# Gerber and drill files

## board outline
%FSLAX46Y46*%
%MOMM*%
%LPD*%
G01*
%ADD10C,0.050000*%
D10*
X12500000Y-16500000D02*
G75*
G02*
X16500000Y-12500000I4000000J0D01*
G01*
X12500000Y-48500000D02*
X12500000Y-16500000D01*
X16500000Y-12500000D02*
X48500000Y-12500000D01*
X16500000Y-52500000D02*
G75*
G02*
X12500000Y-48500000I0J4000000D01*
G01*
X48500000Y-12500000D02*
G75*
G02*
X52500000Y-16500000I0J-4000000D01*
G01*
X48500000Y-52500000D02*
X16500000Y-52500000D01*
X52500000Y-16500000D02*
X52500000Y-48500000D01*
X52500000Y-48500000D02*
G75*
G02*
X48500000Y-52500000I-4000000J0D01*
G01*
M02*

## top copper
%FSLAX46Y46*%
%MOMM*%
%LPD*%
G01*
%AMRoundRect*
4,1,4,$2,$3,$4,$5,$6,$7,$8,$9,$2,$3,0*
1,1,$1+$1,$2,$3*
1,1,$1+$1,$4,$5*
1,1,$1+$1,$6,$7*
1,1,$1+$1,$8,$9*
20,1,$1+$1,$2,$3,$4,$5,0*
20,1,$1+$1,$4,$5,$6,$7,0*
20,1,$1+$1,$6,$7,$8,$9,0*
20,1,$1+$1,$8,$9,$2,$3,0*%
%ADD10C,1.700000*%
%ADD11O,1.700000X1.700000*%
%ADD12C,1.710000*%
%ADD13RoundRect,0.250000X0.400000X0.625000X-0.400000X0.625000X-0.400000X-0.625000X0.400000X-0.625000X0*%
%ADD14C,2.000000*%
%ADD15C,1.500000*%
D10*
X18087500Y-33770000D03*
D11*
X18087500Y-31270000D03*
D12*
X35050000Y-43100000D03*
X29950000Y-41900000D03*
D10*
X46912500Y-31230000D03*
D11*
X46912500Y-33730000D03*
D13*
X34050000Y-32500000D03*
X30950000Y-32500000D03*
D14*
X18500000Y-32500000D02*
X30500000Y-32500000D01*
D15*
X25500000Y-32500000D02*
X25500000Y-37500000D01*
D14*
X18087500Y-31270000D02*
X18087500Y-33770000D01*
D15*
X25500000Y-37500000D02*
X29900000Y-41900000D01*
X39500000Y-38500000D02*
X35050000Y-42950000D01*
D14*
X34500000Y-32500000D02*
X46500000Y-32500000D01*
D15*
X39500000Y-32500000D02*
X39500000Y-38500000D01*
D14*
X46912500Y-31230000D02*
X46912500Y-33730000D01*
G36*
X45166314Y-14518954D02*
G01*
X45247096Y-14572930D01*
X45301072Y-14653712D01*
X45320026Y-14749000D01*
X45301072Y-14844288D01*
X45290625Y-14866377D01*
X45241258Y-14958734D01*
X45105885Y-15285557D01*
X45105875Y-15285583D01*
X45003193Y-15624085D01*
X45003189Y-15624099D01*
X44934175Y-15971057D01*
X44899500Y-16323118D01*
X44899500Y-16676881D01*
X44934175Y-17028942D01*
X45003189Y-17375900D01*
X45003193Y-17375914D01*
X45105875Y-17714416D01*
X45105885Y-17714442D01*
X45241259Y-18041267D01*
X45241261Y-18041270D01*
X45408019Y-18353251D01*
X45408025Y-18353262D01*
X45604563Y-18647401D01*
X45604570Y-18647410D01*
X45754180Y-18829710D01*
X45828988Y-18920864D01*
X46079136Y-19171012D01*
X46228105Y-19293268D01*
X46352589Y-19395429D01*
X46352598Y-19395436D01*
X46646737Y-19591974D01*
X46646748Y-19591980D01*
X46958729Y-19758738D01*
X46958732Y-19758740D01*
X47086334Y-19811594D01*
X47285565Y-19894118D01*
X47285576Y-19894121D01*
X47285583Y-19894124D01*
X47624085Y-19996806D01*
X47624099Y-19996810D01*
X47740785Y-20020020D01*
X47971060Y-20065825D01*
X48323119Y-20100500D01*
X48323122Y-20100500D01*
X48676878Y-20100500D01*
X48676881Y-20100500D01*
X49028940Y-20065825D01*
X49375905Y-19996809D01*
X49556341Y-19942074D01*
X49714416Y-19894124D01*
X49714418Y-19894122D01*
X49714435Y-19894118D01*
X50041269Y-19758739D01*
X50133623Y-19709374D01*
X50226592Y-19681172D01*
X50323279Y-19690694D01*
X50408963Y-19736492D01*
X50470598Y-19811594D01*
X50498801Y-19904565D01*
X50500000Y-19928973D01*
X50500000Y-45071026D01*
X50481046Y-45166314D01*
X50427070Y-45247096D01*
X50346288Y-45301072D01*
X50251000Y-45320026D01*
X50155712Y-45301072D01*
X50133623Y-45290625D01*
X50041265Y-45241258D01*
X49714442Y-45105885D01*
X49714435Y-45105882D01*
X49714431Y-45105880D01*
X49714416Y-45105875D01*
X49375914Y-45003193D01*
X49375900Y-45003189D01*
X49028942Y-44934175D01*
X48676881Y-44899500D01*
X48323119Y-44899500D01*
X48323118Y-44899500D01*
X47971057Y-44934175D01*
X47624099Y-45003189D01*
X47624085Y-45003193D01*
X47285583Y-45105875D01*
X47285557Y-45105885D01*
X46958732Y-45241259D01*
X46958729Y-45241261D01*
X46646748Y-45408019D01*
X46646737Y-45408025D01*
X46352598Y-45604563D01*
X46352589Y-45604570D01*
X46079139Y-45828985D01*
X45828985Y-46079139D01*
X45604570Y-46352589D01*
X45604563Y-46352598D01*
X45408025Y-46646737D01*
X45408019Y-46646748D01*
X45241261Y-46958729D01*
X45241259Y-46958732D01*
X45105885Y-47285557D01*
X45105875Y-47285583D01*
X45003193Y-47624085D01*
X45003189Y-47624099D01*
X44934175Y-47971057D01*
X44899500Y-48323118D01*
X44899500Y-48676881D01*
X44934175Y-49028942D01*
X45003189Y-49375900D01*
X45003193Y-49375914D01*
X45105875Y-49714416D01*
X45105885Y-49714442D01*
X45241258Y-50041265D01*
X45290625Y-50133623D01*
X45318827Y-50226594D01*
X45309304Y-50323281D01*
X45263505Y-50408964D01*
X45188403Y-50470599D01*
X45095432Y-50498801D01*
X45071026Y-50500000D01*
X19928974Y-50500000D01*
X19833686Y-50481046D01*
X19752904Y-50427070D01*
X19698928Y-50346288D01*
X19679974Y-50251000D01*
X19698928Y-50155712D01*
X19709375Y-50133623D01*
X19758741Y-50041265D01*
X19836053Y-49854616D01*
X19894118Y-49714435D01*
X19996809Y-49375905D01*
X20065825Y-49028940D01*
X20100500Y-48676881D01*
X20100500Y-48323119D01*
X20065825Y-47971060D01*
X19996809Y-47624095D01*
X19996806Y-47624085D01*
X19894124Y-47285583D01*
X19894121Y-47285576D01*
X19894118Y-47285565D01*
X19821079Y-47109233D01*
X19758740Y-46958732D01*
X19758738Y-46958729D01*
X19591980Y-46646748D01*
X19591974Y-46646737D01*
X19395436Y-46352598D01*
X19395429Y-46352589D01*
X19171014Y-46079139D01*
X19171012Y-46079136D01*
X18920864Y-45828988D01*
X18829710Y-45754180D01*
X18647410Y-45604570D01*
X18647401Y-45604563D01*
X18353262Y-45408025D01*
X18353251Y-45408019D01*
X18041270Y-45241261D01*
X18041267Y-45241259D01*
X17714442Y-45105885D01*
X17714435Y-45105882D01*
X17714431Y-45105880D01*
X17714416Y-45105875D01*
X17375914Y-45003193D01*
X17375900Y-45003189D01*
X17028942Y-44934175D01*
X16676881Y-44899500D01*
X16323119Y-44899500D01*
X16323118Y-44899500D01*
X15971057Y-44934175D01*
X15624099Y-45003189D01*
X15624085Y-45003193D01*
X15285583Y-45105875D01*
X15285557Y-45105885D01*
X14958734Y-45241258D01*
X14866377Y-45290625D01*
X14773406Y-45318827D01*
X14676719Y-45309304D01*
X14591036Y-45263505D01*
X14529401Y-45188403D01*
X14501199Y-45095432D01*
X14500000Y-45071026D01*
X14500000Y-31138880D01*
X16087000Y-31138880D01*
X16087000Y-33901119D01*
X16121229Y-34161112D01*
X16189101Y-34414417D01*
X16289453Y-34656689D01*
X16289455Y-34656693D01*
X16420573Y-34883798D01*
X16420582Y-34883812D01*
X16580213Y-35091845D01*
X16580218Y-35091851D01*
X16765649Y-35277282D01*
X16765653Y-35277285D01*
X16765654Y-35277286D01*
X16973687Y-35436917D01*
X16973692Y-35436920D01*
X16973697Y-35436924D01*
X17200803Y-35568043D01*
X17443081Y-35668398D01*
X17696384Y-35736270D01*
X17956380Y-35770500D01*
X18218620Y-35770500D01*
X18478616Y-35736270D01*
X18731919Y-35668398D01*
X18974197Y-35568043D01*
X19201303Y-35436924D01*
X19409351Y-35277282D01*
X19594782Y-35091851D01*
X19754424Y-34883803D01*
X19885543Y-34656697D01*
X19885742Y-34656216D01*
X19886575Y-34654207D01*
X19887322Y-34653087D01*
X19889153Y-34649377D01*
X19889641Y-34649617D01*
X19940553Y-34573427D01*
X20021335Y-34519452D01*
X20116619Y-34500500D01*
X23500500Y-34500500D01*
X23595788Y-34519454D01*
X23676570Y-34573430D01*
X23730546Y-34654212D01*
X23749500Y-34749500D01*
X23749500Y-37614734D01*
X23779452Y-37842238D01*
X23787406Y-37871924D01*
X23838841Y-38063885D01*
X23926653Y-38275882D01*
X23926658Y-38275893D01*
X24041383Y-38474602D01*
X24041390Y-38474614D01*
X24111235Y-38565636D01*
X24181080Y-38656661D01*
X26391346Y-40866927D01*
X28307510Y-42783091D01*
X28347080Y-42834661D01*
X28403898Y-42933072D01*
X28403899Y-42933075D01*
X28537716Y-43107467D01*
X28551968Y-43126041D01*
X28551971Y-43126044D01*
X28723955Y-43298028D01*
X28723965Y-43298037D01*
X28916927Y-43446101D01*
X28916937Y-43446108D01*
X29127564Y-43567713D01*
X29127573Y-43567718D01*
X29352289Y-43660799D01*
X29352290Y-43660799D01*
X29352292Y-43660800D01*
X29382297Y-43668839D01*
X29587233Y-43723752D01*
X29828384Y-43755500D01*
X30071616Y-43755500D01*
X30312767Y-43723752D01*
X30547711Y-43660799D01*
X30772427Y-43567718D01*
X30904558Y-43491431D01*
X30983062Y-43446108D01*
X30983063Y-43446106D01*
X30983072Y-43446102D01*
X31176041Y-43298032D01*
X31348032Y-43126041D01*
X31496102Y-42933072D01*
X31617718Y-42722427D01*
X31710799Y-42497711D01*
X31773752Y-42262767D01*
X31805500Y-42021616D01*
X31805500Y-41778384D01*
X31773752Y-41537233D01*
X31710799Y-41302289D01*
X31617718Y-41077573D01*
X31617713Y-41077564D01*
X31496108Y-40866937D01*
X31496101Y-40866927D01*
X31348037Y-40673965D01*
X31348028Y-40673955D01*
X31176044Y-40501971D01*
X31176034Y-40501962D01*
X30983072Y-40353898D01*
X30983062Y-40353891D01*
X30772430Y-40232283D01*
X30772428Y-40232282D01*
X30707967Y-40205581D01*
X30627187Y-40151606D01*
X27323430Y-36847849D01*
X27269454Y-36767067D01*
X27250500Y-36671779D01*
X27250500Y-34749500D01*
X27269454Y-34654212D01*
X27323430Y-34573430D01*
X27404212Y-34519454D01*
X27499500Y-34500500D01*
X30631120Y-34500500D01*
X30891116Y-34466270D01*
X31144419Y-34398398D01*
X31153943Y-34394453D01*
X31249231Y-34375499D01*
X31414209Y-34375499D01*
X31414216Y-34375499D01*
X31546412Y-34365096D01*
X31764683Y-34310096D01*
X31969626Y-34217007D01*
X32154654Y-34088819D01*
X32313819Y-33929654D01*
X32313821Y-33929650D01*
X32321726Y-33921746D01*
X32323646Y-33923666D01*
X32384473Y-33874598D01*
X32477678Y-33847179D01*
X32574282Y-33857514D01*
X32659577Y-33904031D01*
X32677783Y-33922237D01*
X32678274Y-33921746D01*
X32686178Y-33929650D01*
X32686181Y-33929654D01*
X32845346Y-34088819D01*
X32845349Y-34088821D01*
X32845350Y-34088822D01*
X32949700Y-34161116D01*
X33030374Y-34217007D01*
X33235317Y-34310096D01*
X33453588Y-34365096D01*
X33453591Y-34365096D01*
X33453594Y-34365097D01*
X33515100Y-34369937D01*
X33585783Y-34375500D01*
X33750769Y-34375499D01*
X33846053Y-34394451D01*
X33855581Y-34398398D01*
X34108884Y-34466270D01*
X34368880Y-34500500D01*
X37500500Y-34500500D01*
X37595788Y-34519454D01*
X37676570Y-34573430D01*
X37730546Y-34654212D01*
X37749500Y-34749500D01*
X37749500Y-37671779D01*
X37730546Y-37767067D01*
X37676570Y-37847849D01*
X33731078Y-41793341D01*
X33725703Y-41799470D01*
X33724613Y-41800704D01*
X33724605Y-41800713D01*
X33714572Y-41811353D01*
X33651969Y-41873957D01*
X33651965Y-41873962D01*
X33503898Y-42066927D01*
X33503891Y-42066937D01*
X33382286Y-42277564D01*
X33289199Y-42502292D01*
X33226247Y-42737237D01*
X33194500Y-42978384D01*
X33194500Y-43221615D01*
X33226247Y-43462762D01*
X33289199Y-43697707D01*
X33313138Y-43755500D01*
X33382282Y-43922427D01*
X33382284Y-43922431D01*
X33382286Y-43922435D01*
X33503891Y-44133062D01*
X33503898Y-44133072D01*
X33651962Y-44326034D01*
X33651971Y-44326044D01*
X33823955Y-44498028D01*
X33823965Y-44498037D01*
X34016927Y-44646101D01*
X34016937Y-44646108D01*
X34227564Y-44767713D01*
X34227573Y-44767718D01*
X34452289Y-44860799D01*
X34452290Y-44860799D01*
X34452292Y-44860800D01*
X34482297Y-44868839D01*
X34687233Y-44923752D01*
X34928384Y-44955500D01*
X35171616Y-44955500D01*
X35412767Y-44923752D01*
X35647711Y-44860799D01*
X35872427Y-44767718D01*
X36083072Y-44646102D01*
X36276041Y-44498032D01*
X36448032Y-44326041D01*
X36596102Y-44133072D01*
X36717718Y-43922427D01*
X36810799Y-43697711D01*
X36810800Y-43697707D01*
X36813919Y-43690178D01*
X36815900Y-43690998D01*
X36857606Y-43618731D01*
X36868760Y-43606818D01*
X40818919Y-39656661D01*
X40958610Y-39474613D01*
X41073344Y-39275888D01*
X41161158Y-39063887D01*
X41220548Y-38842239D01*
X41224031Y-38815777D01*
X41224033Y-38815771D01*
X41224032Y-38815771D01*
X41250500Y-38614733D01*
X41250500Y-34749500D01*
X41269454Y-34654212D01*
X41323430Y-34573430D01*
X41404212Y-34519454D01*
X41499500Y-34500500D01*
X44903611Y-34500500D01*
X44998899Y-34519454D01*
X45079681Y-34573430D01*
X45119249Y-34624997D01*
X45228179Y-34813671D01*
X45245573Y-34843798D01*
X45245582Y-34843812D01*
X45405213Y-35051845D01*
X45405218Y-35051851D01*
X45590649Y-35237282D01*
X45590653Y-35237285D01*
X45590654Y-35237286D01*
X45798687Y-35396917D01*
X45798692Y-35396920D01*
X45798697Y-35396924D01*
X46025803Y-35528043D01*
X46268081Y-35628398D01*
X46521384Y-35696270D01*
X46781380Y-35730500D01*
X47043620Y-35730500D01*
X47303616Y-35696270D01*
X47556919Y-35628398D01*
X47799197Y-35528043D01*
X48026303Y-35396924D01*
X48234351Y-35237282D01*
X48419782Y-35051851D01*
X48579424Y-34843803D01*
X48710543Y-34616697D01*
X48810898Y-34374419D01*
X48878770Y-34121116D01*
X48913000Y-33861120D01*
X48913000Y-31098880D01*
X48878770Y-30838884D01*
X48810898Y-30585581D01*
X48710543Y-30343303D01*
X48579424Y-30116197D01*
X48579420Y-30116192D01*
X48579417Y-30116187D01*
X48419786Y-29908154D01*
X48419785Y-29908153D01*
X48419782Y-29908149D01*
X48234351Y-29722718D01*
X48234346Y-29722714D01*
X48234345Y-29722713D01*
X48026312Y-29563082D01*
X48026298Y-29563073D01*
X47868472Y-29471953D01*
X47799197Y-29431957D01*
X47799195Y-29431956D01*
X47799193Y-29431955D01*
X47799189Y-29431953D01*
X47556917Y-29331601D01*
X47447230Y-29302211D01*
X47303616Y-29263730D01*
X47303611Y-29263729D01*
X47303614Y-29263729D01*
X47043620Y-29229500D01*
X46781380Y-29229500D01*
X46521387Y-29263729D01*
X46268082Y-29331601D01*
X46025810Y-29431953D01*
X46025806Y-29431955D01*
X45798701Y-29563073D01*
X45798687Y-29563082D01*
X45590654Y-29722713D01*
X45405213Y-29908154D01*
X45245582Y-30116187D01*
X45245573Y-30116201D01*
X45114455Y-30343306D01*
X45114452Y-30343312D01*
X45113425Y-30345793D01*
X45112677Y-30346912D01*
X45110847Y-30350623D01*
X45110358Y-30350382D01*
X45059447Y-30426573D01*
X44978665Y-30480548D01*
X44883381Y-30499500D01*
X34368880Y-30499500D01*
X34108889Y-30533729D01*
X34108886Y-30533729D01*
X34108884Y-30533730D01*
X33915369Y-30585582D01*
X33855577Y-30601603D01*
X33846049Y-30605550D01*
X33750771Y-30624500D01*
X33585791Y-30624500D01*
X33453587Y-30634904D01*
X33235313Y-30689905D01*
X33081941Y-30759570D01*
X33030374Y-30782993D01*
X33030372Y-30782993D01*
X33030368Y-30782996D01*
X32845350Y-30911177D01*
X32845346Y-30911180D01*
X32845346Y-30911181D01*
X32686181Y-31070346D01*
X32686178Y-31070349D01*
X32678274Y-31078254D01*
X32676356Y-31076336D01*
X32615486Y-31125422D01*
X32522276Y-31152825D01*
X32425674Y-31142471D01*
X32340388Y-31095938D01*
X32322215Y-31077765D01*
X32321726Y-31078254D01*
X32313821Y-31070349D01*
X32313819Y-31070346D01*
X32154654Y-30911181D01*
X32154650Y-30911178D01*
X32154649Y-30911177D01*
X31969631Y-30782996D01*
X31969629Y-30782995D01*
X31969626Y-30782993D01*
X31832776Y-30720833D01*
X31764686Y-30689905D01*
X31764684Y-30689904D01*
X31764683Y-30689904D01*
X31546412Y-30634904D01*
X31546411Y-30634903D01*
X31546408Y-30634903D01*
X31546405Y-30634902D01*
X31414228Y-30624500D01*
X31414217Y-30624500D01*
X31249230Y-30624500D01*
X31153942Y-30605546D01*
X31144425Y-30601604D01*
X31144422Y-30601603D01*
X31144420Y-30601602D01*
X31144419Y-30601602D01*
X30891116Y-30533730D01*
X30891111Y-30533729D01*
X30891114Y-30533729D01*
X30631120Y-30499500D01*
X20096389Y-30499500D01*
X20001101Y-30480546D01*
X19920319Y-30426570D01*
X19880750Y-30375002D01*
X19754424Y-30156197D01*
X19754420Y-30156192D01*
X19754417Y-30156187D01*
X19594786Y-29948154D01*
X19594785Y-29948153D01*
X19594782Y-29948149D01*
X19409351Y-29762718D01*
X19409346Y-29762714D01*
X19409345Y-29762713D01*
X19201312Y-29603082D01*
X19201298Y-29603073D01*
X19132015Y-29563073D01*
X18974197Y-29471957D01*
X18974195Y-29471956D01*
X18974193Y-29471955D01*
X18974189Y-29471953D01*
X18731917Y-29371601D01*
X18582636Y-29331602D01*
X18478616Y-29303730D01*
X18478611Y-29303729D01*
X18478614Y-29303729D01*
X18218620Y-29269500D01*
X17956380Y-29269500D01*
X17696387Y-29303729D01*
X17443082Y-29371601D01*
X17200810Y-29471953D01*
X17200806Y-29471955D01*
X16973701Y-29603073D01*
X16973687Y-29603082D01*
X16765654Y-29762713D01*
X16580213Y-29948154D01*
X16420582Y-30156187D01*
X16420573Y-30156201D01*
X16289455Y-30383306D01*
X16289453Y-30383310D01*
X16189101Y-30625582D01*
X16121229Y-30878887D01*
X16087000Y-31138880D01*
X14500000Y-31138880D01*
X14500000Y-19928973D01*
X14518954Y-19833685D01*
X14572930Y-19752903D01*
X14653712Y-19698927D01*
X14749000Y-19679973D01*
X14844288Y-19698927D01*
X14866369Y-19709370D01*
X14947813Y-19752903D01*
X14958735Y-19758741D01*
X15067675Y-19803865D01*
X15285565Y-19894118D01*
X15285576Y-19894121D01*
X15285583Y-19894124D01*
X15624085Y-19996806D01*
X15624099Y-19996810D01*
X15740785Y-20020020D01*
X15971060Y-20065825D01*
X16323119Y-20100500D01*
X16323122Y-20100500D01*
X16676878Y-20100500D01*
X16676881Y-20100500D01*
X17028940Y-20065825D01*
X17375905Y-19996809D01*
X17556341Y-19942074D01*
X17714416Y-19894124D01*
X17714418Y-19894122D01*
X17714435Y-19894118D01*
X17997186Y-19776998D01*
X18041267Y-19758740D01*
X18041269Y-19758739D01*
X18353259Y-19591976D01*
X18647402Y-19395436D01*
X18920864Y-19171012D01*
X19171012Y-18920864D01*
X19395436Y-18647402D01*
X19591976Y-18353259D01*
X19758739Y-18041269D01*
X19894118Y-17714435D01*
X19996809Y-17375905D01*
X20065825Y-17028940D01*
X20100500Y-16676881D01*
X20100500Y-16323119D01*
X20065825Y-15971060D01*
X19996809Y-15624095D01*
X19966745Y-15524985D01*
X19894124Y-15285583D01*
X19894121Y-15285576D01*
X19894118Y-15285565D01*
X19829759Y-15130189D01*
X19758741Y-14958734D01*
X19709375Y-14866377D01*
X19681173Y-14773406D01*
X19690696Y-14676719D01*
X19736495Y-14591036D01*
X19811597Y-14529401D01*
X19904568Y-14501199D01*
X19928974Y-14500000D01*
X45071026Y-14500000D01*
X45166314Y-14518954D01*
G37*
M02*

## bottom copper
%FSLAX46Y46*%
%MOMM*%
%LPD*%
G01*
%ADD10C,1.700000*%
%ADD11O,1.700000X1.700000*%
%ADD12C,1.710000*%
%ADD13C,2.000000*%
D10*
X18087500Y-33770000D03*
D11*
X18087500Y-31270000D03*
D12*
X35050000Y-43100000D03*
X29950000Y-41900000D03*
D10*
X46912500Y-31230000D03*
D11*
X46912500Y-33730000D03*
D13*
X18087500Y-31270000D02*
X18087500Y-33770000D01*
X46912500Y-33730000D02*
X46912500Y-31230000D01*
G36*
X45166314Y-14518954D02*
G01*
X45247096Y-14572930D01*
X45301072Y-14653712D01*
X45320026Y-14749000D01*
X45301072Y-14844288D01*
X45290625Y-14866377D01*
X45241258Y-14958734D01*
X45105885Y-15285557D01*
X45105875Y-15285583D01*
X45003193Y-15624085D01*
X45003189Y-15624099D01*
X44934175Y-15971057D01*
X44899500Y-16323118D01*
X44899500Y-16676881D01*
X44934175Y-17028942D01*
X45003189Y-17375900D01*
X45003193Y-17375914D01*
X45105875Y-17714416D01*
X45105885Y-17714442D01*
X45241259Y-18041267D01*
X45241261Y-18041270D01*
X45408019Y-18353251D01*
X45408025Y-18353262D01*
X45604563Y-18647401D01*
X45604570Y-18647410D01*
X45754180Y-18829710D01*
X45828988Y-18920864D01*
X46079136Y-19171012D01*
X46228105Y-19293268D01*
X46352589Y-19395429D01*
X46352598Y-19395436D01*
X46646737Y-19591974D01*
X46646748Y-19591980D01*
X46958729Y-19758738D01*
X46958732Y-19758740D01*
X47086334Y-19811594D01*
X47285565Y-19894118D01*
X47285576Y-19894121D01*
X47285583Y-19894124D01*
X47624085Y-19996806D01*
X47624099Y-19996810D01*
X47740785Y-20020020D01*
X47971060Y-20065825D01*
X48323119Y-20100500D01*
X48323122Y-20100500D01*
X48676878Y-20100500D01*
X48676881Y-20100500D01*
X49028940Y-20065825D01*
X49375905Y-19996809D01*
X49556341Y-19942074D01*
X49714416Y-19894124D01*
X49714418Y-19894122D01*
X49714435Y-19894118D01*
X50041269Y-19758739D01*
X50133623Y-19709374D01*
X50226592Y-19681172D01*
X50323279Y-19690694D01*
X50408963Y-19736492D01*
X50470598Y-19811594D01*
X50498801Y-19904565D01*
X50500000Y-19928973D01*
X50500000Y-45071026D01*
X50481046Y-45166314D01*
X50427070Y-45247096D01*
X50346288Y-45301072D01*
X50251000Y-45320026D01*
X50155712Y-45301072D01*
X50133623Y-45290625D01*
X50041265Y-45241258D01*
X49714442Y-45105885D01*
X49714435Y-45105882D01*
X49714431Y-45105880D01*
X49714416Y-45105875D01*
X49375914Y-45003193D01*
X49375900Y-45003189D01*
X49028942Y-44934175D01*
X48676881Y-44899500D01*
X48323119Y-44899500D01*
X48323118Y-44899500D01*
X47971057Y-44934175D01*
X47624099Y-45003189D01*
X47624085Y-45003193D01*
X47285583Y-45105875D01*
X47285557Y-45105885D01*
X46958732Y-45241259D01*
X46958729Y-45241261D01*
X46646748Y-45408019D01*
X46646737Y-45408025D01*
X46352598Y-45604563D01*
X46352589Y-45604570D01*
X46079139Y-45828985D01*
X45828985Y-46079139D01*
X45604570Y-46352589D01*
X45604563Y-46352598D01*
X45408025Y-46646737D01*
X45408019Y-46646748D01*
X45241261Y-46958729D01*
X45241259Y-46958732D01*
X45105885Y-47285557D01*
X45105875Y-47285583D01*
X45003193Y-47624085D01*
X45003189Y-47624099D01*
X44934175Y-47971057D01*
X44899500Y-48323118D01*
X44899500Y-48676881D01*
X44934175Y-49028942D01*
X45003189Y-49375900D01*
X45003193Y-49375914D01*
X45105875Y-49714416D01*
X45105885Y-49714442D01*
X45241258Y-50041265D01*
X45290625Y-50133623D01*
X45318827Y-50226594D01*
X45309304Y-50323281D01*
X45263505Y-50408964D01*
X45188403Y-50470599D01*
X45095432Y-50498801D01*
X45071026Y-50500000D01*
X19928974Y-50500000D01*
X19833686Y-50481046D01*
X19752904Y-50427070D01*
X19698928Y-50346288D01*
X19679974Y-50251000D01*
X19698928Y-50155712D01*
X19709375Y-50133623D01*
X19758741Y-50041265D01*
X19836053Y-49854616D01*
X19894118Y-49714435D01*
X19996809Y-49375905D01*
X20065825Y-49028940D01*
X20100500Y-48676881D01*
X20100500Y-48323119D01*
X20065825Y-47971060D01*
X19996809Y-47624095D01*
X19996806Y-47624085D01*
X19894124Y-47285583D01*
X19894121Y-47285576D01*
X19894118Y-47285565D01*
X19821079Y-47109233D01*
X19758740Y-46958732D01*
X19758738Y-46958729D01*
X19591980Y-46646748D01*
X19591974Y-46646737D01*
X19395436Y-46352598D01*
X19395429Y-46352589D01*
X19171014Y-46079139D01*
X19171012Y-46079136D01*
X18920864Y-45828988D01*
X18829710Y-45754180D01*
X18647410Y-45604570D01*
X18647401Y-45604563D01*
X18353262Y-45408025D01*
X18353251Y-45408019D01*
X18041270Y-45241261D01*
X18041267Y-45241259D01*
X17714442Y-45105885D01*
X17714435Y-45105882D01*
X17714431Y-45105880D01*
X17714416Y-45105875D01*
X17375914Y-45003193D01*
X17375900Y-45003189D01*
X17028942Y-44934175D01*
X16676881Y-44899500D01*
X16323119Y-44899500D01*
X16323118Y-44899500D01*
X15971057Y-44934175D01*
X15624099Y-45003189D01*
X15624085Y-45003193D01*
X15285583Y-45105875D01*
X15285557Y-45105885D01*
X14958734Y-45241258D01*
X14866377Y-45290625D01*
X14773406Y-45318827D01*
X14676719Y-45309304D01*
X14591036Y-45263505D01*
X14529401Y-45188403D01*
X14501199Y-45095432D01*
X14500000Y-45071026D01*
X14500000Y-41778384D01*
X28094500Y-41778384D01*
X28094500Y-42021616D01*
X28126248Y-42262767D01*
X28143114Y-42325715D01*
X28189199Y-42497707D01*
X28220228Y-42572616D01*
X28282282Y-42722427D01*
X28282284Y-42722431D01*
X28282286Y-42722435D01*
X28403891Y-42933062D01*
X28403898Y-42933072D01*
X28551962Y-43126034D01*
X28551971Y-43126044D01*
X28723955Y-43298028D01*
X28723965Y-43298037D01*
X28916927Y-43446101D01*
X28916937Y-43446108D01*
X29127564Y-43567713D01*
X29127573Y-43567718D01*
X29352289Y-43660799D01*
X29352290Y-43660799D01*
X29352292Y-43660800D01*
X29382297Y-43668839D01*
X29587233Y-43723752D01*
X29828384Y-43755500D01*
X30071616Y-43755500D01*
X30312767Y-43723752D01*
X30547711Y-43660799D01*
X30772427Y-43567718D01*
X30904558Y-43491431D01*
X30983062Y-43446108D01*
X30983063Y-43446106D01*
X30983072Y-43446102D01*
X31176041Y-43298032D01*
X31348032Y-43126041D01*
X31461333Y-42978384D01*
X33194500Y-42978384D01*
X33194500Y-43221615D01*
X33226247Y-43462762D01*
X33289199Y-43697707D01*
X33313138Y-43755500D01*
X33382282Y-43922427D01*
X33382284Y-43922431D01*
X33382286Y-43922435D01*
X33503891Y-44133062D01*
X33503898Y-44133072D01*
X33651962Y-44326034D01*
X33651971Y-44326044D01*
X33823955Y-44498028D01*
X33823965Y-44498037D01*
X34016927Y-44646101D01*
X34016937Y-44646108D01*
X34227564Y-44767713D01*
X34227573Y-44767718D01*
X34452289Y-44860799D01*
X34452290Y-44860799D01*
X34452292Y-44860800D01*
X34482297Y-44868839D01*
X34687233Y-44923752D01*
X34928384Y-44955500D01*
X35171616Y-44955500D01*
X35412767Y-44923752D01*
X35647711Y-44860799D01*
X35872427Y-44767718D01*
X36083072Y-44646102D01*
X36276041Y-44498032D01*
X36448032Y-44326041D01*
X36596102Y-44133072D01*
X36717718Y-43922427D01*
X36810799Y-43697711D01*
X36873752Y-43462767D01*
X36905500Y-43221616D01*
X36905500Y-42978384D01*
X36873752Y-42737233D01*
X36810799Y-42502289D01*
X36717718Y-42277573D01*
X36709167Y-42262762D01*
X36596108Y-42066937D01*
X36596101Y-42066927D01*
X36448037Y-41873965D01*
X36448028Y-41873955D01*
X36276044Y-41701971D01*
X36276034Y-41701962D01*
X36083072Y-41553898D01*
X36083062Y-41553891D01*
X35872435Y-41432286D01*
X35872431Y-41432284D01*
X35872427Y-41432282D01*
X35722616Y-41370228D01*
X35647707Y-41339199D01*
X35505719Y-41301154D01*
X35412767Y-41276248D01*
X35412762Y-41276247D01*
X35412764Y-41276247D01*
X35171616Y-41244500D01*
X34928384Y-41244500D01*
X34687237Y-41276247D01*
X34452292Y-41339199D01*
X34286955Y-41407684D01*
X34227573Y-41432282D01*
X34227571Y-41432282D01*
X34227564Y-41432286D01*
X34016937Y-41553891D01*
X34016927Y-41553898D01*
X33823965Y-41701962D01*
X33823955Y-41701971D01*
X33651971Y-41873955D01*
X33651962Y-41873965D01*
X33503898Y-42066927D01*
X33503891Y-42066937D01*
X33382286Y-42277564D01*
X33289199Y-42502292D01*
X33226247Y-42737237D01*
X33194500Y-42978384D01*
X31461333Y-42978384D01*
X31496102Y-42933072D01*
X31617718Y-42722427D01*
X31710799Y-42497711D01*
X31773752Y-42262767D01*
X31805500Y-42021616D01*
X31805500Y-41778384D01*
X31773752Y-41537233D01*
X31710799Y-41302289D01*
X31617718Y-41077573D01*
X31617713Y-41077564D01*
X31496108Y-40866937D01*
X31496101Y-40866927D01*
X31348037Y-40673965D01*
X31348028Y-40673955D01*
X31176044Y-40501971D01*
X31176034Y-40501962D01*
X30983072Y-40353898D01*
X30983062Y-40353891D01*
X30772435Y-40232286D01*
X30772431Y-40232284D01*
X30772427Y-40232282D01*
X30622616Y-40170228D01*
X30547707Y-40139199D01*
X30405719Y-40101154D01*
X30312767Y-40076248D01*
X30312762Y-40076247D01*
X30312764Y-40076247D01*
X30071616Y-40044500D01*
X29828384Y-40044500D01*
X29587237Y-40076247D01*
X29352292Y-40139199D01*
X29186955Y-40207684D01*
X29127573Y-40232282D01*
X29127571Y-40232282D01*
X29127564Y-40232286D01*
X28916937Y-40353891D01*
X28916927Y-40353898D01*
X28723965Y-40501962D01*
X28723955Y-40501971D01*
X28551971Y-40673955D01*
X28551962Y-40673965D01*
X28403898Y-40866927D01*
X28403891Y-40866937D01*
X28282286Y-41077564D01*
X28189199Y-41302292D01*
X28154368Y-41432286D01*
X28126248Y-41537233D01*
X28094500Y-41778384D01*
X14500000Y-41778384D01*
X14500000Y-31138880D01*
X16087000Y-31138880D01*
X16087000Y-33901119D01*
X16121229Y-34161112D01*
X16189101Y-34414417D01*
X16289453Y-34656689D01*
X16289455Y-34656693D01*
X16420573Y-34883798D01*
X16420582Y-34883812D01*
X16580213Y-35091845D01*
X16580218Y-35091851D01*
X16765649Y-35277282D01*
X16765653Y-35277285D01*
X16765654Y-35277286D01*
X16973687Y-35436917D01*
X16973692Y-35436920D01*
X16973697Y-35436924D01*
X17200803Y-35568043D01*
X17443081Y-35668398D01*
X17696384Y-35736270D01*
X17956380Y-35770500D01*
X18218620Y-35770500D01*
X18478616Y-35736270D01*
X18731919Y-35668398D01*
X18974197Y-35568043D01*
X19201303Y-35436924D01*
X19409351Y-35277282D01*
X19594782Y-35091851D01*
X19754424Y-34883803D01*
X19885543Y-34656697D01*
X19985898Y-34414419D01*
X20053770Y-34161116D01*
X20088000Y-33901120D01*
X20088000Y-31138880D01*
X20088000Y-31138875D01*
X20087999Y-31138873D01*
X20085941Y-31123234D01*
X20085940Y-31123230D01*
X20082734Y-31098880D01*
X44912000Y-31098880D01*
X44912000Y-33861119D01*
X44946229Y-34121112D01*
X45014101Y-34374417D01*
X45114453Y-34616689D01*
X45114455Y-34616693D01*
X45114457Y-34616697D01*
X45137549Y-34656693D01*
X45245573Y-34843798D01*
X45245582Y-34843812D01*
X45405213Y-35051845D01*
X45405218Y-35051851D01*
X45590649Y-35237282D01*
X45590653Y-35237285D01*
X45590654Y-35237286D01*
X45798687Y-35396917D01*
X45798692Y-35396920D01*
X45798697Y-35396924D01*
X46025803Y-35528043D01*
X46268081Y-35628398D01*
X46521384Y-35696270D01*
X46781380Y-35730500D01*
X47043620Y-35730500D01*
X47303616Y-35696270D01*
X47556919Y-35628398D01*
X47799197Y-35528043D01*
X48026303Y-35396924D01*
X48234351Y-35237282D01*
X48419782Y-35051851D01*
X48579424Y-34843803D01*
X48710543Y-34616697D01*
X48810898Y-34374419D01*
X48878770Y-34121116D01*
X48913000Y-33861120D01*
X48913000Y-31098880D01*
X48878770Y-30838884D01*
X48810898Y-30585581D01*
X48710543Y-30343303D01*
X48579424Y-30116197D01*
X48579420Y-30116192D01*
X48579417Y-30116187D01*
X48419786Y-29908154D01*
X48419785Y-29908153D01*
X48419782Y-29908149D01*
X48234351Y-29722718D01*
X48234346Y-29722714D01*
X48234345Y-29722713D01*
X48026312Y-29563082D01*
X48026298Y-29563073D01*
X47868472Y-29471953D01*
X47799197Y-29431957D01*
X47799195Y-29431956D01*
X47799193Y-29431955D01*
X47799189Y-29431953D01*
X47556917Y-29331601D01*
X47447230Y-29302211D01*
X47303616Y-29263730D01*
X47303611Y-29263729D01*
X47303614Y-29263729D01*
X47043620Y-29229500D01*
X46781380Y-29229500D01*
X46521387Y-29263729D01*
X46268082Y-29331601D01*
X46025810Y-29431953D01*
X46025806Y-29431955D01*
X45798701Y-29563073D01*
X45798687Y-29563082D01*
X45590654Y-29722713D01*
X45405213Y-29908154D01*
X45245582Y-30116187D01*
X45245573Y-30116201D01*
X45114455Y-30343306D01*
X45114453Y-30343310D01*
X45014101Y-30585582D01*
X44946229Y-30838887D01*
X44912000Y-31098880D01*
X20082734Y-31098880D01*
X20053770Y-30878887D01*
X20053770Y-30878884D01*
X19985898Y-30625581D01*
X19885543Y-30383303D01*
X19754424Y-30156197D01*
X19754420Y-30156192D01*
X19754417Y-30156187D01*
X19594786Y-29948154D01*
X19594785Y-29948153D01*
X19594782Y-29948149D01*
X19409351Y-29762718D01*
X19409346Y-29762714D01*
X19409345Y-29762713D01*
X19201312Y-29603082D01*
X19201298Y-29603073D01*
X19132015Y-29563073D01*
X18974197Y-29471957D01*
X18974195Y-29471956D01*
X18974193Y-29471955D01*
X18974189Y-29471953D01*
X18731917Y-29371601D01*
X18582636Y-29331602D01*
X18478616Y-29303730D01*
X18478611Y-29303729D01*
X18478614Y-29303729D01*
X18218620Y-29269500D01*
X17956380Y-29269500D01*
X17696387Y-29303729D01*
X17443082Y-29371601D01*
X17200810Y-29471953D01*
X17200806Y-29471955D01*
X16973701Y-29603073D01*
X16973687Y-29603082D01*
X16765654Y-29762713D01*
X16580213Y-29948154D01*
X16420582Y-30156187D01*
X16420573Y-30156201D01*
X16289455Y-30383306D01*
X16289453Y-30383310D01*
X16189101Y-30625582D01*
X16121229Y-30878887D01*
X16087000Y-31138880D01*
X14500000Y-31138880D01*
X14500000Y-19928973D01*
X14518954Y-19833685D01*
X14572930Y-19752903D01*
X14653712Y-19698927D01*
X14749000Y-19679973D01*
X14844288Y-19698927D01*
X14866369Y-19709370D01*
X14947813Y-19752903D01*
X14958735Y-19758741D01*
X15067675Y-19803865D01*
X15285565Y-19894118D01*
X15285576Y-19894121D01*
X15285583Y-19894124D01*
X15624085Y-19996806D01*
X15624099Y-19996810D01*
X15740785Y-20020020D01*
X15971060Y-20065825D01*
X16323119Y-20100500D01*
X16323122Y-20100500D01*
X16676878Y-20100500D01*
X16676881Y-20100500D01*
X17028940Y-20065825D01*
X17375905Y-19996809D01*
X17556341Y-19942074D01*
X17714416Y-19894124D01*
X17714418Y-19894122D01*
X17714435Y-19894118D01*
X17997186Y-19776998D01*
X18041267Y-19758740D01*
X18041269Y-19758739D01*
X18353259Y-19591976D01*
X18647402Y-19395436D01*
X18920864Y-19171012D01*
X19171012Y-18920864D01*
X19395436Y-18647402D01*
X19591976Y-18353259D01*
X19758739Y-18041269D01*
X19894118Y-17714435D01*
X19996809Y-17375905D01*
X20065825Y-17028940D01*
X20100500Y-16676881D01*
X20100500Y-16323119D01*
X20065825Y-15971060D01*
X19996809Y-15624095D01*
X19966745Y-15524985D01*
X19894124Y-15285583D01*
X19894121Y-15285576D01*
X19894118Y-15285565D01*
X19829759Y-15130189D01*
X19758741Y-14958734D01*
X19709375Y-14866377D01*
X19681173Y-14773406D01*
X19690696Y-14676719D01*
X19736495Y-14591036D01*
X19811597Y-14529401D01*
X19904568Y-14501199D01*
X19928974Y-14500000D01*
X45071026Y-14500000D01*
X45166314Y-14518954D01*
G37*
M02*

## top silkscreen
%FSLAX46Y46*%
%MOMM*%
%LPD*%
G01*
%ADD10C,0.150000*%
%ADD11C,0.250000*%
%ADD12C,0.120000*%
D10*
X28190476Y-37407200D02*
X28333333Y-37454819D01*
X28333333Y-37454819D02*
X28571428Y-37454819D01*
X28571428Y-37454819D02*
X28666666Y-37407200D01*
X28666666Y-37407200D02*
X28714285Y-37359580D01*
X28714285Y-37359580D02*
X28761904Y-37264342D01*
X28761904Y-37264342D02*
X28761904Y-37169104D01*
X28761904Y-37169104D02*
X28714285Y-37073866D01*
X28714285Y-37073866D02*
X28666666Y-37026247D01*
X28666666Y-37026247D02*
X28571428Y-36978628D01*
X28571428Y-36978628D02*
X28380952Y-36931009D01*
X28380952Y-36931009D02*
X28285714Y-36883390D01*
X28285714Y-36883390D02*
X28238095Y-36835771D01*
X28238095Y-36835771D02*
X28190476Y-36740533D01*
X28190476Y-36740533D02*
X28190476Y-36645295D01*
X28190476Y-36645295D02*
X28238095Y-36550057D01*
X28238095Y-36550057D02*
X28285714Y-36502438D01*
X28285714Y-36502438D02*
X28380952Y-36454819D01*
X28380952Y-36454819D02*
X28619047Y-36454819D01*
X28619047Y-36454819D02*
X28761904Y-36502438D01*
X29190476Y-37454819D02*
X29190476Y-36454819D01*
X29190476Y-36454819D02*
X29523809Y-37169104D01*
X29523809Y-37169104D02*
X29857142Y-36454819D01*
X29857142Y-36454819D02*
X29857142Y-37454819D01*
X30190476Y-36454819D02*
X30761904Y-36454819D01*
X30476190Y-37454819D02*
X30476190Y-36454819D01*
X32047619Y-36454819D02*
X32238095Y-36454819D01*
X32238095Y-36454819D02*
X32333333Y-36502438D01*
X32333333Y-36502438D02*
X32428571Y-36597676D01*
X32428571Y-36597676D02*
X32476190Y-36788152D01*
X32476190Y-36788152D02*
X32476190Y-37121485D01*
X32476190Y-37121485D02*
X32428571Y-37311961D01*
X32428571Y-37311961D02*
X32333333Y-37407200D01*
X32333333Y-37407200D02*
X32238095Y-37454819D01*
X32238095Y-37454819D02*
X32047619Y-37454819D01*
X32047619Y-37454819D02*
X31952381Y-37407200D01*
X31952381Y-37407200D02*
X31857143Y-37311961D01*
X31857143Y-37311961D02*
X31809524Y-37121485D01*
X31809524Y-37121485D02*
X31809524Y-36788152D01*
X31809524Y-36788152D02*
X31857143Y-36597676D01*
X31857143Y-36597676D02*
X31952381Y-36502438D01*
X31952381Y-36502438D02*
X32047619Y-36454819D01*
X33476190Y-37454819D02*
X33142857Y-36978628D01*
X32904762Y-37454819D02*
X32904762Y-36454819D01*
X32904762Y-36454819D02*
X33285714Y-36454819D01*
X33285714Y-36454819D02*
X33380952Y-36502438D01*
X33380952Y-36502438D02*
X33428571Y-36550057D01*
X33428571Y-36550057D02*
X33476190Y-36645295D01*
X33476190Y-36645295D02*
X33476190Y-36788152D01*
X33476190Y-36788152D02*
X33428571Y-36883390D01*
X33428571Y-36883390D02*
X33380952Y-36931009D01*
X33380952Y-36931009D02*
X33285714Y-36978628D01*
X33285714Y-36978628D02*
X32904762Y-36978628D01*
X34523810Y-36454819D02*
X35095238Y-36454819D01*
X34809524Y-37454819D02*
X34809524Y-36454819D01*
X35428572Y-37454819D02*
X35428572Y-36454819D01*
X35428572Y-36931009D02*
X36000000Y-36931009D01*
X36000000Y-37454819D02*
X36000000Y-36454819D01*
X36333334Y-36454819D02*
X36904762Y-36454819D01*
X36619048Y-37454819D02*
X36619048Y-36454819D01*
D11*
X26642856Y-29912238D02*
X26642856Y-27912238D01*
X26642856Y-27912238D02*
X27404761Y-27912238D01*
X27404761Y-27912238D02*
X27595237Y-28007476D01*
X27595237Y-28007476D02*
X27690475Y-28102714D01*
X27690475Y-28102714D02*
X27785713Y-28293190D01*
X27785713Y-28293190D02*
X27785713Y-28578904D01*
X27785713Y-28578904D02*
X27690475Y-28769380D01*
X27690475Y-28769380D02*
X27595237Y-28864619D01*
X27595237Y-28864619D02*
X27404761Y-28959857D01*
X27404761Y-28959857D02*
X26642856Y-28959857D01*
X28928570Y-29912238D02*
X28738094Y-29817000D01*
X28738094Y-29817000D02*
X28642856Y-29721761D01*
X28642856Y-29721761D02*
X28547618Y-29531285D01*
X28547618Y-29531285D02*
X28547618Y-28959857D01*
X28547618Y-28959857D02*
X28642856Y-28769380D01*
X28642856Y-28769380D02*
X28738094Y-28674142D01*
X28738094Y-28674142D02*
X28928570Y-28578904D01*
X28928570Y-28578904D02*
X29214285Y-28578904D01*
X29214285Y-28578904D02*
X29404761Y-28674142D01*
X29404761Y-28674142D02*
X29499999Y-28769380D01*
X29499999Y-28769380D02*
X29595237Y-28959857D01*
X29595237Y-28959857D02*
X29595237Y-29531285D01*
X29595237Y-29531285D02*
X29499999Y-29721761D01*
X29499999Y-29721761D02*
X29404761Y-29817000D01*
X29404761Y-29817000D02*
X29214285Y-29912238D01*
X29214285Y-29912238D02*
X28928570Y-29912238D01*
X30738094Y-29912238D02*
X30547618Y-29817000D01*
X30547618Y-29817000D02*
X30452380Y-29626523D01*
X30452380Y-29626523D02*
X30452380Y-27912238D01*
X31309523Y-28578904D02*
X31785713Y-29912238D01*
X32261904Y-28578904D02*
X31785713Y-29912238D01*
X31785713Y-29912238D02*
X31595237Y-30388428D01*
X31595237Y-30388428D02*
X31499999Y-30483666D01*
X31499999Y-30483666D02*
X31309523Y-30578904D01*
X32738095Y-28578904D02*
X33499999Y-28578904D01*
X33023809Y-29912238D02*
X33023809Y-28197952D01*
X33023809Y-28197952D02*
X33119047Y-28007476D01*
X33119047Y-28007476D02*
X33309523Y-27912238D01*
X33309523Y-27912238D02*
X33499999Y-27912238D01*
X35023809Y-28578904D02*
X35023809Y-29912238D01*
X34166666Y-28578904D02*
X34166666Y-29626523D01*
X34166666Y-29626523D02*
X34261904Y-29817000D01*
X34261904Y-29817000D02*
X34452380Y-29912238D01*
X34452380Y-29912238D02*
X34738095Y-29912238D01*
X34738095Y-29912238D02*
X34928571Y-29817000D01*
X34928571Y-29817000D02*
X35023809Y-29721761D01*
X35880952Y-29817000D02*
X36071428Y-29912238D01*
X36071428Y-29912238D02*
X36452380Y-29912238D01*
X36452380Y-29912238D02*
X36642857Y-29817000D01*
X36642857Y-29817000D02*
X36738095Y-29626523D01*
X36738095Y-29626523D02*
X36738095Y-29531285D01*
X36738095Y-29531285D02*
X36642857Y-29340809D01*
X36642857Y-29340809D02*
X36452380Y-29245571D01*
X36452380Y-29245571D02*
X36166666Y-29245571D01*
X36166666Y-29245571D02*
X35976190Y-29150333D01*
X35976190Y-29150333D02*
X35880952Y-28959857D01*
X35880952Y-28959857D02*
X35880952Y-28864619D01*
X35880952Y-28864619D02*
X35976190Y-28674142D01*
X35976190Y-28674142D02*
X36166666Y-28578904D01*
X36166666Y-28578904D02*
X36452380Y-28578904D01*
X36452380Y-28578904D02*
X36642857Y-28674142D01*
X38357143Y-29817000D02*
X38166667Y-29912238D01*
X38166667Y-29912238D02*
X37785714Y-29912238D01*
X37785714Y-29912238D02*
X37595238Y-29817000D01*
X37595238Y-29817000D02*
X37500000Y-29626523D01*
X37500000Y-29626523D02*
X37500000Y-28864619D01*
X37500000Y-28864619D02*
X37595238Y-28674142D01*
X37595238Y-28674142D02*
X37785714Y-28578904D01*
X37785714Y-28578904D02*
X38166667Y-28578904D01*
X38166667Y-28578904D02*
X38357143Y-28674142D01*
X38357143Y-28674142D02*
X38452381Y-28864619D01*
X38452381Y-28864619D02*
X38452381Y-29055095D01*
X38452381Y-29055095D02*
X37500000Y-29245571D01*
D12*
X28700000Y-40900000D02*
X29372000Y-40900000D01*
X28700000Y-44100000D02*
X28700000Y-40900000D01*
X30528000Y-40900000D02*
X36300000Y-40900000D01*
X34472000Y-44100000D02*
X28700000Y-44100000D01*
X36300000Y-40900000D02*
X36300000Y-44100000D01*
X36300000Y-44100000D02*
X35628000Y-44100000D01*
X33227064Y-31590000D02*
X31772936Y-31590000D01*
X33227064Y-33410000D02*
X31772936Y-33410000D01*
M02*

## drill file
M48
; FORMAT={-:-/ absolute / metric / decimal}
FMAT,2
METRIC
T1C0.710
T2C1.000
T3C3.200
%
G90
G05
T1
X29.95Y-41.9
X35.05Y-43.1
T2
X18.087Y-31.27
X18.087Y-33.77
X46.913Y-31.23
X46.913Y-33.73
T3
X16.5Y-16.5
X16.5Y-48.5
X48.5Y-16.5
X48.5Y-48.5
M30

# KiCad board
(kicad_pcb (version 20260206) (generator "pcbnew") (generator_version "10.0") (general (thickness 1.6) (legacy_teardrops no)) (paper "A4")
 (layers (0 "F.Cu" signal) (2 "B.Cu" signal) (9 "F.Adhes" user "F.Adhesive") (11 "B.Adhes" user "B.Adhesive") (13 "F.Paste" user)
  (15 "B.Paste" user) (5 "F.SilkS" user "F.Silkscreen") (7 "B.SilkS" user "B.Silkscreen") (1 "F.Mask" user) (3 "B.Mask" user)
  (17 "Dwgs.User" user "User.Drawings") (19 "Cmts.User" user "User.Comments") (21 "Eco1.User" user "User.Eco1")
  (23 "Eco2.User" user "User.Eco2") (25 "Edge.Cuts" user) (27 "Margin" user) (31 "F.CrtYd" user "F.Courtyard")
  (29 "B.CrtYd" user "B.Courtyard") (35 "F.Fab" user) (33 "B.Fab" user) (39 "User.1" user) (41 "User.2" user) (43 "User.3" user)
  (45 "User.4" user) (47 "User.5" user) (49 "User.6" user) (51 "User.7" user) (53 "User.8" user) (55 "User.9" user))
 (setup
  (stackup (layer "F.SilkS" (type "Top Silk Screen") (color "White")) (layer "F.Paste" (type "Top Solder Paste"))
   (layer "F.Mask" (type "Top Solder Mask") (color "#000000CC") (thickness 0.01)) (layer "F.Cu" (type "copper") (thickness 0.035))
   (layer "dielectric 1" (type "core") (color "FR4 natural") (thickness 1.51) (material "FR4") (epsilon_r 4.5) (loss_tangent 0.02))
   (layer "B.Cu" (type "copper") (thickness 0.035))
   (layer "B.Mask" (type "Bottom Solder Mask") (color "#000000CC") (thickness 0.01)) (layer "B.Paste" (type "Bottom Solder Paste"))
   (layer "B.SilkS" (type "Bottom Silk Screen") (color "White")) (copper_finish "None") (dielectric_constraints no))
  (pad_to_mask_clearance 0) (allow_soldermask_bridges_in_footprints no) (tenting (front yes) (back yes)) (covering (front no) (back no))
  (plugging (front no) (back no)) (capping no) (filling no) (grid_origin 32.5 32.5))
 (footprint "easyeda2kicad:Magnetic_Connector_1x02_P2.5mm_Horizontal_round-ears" (layer "F.Cu") (at 17.9875 32.5 180)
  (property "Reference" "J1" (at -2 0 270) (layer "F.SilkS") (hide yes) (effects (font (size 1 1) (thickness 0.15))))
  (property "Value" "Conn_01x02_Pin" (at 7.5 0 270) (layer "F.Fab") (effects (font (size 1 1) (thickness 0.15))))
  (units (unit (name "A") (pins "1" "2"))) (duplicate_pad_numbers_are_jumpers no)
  (pad "1" thru_hole circle (at -0.1 -1.27 180) (size 1.7 1.7) (drill 1) (layers "*.Cu" "*.Mask") (remove_unused_layers no)
   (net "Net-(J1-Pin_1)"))
  (pad "2" thru_hole oval (at -0.1 1.23 180) (size 1.7 1.7) (drill 1) (layers "*.Cu" "*.Mask") (remove_unused_layers no)
   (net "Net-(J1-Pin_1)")))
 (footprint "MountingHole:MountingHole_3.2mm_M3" (layer "F.Cu") (at 48.5 16.5)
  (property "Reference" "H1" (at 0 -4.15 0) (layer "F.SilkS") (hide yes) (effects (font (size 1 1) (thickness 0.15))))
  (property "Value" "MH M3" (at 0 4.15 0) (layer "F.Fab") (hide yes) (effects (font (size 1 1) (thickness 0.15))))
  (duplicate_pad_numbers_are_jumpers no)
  (pad "" np_thru_hole circle (at 0 0) (size 3.2 3.2) (drill 3.2) (layers "*.Cu" "*.Mask") (clearance 2)))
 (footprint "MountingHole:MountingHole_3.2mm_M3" (layer "F.Cu") (at 48.5 48.5)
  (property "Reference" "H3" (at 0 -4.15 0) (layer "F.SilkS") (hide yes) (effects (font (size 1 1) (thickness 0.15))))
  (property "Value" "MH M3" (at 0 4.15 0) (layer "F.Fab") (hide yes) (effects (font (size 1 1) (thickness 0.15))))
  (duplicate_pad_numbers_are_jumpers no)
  (pad "" np_thru_hole circle (at 0 0) (size 3.2 3.2) (drill 3.2) (layers "*.Cu" "*.Mask") (clearance 2)))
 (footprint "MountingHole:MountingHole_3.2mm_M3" (layer "F.Cu") (at 16.5 16.5)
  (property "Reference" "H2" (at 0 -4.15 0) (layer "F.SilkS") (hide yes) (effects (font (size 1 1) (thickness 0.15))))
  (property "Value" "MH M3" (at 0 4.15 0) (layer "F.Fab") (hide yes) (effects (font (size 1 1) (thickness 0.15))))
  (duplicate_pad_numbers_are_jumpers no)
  (pad "" np_thru_hole circle (at 0 0) (size 3.2 3.2) (drill 3.2) (layers "*.Cu" "*.Mask") (clearance 2)))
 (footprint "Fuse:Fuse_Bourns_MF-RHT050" (layer "F.Cu") (at 35.05 43.1 180)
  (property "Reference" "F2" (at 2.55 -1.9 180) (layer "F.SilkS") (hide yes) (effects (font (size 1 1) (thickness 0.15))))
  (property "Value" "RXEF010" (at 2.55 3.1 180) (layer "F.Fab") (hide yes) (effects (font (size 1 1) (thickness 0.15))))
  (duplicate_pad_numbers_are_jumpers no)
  (fp_line (start 6.35 2.2) (end 5.678 2.2) (stroke (width 0.12) (type solid)) (layer "F.SilkS"))
  (fp_line (start 6.35 -1) (end 6.35 2.2) (stroke (width 0.12) (type solid)) (layer "F.SilkS"))
  (fp_line (start 4.522 2.2) (end -1.25 2.2) (stroke (width 0.12) (type solid)) (layer "F.SilkS"))
  (fp_line (start 0.578 -1) (end 6.35 -1) (stroke (width 0.12) (type solid)) (layer "F.SilkS"))
  (fp_line (start -1.25 2.2) (end -1.25 -1) (stroke (width 0.12) (type solid)) (layer "F.SilkS"))
  (fp_line (start -1.25 -1) (end -0.578 -1) (stroke (width 0.12) (type solid)) (layer "F.SilkS"))
  (pad "1" thru_hole circle (at 0 0 180) (size 1.71 1.71) (drill 0.71) (layers "*.Cu" "*.Mask") (remove_unused_layers no)
   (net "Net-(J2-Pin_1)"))
  (pad "2" thru_hole circle (at 5.1 1.2 180) (size 1.71 1.71) (drill 0.71) (layers "*.Cu" "*.Mask") (remove_unused_layers no)
   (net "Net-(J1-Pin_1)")))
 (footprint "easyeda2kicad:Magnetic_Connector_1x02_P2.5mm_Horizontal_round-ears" (layer "F.Cu") (at 47.0125 32.5)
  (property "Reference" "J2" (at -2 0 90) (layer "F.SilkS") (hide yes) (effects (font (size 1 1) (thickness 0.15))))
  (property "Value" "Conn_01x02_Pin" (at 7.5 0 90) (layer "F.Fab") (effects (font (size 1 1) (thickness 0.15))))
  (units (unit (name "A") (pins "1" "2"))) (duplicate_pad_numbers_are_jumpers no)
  (pad "1" thru_hole circle (at -0.1 -1.27) (size 1.7 1.7) (drill 1) (layers "*.Cu" "*.Mask") (remove_unused_layers no)
   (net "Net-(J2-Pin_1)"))
  (pad "2" thru_hole oval (at -0.1 1.23) (size 1.7 1.7) (drill 1) (layers "*.Cu" "*.Mask") (remove_unused_layers no) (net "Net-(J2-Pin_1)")))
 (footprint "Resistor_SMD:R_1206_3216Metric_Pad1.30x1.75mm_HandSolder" (layer "F.Cu") (at 32.5 32.5 180)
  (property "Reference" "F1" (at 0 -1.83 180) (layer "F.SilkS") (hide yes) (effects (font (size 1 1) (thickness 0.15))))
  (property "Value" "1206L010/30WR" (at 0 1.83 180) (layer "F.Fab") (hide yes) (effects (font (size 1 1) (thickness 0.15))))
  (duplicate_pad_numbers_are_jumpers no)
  (fp_line (start -0.727064 0.91) (end 0.727064 0.91) (stroke (width 0.12) (type solid)) (layer "F.SilkS"))
  (fp_line (start -0.727064 -0.91) (end 0.727064 -0.91) (stroke (width 0.12) (type solid)) (layer "F.SilkS"))
  (pad "1" smd roundrect (at -1.55 0 180) (size 1.3 1.75) (layers "F.Cu" "F.Mask" "F.Paste") (roundrect_rratio 0.192308)
   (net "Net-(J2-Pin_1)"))
  (pad "2" smd roundrect (at 1.55 0 180) (size 1.3 1.75) (layers "F.Cu" "F.Mask" "F.Paste") (roundrect_rratio 0.192308)
   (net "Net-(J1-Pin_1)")))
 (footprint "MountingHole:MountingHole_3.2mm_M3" (layer "F.Cu") (at 16.5 48.5)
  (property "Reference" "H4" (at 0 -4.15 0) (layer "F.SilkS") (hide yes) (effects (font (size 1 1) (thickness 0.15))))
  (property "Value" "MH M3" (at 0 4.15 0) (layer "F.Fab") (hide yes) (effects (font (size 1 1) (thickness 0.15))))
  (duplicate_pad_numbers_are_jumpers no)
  (pad "" np_thru_hole circle (at 0 0) (size 3.2 3.2) (drill 3.2) (layers "*.Cu" "*.Mask") (clearance 2)))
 (gr_arc (start 12.5 16.5) (mid 13.671573 13.671573) (end 16.5 12.5) (stroke (width 0.05) (type default)) (layer "Edge.Cuts"))
 (gr_line (start 12.5 48.5) (end 12.5 16.5) (stroke (width 0.05) (type default)) (layer "Edge.Cuts"))
 (gr_line (start 16.5 12.5) (end 48.5 12.5) (stroke (width 0.05) (type default)) (layer "Edge.Cuts"))
 (gr_arc (start 16.5 52.5) (mid 13.671573 51.328427) (end 12.5 48.5) (stroke (width 0.05) (type default)) (layer "Edge.Cuts"))
 (gr_arc (start 48.5 12.5) (mid 51.328427 13.671573) (end 52.5 16.5) (stroke (width 0.05) (type default)) (layer "Edge.Cuts"))
 (gr_line (start 48.5 52.5) (end 16.5 52.5) (stroke (width 0.05) (type default)) (layer "Edge.Cuts"))
 (gr_line (start 52.5 16.5) (end 52.5 48.5) (stroke (width 0.05) (type default)) (layer "Edge.Cuts"))
 (gr_arc (start 52.5 48.5) (mid 51.328427 51.328427) (end 48.5 52.5) (stroke (width 0.05) (type default)) (layer "Edge.Cuts"))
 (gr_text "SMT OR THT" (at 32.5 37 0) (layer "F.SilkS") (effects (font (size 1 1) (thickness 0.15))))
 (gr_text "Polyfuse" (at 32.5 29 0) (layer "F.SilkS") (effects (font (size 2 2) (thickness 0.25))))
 (segment (start 18.5 32.5) (end 30.5 32.5) (width 2) (layer "F.Cu") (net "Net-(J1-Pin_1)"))
 (segment (start 25.5 32.5) (end 25.5 37.5) (width 1.5) (layer "F.Cu") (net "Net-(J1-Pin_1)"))
 (segment (start 18.0875 31.27) (end 18.0875 33.77) (width 2) (layer "F.Cu") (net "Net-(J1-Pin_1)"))
 (segment (start 25.5 37.5) (end 29.9 41.9) (width 1.5) (layer "F.Cu") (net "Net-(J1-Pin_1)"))
 (segment (start 18.0875 31.27) (end 18.0875 33.77) (width 2) (layer "B.Cu") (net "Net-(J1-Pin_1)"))
 (segment (start 39.5 38.5) (end 35.05 42.95) (width 1.5) (layer "F.Cu") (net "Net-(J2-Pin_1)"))
 (segment (start 34.5 32.5) (end 46.5 32.5) (width 2) (layer "F.Cu") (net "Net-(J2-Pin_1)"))
 (segment (start 39.5 32.5) (end 39.5 38.5) (width 1.5) (layer "F.Cu") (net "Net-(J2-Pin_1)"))
 (segment (start 46.9125 31.23) (end 46.9125 33.73) (width 2) (layer "F.Cu") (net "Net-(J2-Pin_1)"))
 (segment (start 46.9125 33.73) (end 46.9125 31.23) (width 2) (layer "B.Cu") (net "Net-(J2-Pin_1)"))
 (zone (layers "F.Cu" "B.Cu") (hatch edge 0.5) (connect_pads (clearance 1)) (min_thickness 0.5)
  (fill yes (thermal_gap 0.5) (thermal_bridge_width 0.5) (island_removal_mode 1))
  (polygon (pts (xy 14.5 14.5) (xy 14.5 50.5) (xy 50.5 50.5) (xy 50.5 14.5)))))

